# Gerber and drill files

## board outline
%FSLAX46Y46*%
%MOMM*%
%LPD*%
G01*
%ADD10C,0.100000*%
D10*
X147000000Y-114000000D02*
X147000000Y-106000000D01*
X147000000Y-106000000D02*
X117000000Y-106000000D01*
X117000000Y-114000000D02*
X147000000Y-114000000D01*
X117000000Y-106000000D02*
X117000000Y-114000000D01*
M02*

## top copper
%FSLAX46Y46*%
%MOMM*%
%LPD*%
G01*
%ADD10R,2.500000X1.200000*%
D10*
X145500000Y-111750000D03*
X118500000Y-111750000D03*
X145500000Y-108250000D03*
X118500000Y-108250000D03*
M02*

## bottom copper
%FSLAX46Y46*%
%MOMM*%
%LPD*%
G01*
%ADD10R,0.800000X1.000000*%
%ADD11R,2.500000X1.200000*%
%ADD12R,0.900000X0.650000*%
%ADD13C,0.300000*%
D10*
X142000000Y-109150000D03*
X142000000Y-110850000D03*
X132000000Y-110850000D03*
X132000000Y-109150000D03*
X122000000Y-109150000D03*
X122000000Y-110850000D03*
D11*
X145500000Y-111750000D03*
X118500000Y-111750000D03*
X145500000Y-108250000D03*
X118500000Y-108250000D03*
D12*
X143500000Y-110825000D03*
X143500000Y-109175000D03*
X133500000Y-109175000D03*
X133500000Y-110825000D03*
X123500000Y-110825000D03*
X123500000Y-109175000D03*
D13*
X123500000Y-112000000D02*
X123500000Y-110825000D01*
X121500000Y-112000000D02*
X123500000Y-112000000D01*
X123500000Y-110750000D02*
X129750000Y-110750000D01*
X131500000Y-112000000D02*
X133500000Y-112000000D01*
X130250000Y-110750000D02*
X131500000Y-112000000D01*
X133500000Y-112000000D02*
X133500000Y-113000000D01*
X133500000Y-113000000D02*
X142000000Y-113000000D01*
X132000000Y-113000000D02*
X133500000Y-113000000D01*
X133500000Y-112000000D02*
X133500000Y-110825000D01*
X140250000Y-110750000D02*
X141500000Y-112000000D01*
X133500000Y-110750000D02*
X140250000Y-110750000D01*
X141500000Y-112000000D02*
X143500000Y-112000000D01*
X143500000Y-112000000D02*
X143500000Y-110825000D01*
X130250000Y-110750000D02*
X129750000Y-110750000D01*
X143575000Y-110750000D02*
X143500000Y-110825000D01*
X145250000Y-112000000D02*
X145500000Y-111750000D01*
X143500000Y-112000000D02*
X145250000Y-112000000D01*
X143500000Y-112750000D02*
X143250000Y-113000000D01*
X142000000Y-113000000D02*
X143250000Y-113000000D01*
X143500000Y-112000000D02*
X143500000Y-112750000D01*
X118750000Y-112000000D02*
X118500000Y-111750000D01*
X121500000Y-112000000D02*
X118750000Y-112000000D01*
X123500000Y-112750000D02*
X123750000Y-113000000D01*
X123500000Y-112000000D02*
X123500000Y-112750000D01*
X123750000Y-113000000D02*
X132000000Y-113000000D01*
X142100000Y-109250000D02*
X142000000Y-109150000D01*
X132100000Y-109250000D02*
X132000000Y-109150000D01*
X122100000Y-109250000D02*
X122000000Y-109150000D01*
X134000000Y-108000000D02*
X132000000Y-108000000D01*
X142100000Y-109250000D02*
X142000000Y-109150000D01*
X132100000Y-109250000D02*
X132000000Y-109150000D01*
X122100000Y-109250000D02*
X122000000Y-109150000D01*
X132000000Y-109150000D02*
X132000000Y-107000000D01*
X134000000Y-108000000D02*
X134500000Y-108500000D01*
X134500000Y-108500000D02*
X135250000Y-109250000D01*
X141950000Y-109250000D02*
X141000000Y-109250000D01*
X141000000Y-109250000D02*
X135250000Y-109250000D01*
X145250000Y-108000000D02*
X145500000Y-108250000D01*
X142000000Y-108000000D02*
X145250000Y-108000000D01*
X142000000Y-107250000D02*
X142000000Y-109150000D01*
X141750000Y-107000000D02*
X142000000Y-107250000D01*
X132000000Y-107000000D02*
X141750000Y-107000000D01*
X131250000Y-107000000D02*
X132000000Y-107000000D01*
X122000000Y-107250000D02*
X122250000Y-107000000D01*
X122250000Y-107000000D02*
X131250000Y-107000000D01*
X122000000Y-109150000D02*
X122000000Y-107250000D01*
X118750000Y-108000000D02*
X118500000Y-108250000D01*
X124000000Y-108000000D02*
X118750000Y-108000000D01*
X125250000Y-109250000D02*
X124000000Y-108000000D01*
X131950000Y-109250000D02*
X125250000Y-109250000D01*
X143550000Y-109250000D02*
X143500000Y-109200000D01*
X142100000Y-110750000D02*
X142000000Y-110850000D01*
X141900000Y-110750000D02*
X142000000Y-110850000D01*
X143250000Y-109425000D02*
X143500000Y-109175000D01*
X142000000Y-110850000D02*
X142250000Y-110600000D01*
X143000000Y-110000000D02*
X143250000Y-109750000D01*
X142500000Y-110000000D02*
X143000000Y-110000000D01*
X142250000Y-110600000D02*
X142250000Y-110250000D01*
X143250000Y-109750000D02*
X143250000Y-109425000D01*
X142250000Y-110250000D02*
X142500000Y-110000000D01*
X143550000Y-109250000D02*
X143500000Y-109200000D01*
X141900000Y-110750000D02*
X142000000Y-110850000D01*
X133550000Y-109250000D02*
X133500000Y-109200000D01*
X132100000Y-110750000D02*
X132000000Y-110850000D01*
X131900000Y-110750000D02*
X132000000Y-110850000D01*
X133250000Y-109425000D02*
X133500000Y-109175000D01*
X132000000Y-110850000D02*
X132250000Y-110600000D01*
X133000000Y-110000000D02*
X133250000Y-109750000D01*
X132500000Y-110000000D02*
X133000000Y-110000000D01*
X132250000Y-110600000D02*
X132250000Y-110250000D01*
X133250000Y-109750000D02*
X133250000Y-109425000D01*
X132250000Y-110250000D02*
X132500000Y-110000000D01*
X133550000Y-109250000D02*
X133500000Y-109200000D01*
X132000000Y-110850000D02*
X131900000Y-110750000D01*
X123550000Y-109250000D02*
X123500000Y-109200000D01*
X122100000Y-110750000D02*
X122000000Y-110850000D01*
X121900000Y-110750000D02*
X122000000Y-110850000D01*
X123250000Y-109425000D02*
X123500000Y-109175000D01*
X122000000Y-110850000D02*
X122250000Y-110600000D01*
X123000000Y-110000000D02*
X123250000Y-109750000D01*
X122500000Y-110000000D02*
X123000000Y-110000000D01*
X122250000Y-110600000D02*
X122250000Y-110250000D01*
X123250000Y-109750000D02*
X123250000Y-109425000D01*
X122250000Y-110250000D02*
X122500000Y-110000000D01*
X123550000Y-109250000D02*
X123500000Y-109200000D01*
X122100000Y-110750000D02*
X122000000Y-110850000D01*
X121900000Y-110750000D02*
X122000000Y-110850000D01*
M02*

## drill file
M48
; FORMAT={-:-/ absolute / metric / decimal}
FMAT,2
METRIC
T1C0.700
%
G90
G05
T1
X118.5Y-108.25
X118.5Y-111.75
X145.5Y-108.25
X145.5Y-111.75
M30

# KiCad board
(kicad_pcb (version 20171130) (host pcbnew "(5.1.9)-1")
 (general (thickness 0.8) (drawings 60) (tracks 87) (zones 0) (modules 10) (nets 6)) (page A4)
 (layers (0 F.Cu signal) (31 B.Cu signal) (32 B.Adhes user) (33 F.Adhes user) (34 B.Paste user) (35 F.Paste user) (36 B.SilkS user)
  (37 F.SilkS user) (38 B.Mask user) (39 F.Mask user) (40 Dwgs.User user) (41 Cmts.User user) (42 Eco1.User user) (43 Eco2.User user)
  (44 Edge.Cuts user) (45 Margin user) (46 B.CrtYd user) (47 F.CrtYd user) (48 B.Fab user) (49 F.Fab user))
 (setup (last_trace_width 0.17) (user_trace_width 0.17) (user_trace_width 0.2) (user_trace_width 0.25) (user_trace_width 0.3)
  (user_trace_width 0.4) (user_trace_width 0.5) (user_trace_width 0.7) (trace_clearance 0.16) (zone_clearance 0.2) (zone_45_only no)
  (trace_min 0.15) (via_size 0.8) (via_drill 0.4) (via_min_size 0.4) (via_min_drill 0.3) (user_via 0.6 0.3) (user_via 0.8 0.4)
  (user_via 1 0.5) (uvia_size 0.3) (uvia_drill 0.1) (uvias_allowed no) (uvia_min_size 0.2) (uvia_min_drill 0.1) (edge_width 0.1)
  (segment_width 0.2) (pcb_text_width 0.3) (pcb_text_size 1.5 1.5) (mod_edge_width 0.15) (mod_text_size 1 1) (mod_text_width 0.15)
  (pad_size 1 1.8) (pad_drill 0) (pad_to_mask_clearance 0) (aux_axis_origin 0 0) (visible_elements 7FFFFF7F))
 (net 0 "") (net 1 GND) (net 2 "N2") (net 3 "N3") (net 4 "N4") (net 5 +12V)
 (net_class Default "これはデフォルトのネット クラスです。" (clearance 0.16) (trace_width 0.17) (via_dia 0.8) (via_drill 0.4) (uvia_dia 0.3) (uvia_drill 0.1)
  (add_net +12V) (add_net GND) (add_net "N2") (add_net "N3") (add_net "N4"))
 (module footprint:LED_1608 (layer B.Cu) (at 142 110 270)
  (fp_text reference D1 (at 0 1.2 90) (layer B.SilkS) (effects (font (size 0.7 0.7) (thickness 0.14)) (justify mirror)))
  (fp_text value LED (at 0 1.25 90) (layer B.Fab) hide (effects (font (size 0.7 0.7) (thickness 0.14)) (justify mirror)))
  (pad 1 smd rect (at -0.85 0 270) (size 1 0.8) (layers B.Cu B.Paste B.Mask) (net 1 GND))
  (pad 2 smd rect (at 0.85 0 270) (size 1 0.8) (layers B.Cu B.Paste B.Mask) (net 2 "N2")))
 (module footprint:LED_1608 (layer B.Cu) (at 132 110 270)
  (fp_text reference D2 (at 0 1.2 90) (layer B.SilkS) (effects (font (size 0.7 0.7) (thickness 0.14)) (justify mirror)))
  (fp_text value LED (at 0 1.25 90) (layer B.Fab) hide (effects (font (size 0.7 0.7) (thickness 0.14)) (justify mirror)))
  (pad 2 smd rect (at 0.85 0 270) (size 1 0.8) (layers B.Cu B.Paste B.Mask) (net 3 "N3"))
  (pad 1 smd rect (at -0.85 0 270) (size 1 0.8) (layers B.Cu B.Paste B.Mask) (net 1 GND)))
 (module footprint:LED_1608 (layer B.Cu) (at 122 110 270)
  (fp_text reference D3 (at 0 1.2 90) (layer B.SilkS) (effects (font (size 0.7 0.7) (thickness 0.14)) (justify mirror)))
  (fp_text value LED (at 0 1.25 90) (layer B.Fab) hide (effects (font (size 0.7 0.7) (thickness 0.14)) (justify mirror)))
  (pad 1 smd rect (at -0.85 0 270) (size 1 0.8) (layers B.Cu B.Paste B.Mask) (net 1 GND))
  (pad 2 smd rect (at 0.85 0 270) (size 1 0.8) (layers B.Cu B.Paste B.Mask) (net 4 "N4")))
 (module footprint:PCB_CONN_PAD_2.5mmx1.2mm (layer F.Cu) (at 145.5 111.75)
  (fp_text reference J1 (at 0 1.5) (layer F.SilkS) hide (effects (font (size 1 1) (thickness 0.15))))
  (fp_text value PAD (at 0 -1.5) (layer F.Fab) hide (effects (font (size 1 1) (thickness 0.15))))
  (pad 1 thru_hole rect (at 0 0) (size 2.5 1.2) (drill 0.7) (layers *.Cu *.Mask) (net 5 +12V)))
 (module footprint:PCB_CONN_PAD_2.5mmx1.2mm (layer F.Cu) (at 118.5 111.75)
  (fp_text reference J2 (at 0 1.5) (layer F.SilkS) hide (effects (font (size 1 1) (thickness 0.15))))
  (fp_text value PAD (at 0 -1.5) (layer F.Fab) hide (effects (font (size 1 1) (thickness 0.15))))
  (pad 1 thru_hole rect (at 0 0) (size 2.5 1.2) (drill 0.7) (layers *.Cu *.Mask) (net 5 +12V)))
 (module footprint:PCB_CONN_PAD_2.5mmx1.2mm (layer F.Cu) (at 145.5 108.25)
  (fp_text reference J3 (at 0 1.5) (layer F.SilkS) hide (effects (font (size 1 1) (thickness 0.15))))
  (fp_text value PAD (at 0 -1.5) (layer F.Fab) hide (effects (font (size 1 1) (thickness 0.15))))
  (pad 1 thru_hole rect (at 0 0) (size 2.5 1.2) (drill 0.7) (layers *.Cu *.Mask) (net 1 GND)))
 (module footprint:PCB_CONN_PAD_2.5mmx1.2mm (layer F.Cu) (at 118.5 108.25)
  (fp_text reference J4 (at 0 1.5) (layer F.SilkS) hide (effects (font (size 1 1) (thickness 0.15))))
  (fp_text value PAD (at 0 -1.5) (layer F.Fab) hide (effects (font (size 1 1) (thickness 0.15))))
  (pad 1 thru_hole rect (at 0 0) (size 2.5 1.2) (drill 0.7) (layers *.Cu *.Mask) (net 1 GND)))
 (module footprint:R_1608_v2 (layer B.Cu) (at 143.5 110 90)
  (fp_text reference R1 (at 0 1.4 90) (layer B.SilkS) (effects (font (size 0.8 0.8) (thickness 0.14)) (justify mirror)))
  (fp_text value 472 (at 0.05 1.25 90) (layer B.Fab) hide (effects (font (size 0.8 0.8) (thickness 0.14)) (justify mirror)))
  (pad 1 smd rect (at -0.825 0 90) (size 0.65 0.9) (layers B.Cu B.Paste B.Mask) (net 5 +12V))
  (pad 2 smd rect (at 0.825 0 90) (size 0.65 0.9) (layers B.Cu B.Paste B.Mask) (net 2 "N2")))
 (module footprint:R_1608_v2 (layer B.Cu) (at 133.5 110 90)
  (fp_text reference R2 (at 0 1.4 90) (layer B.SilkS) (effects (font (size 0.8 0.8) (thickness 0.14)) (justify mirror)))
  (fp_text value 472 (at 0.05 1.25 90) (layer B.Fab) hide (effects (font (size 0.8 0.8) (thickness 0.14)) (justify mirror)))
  (pad 2 smd rect (at 0.825 0 90) (size 0.65 0.9) (layers B.Cu B.Paste B.Mask) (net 3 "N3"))
  (pad 1 smd rect (at -0.825 0 90) (size 0.65 0.9) (layers B.Cu B.Paste B.Mask) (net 5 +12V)))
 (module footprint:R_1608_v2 (layer B.Cu) (at 123.5 110 90)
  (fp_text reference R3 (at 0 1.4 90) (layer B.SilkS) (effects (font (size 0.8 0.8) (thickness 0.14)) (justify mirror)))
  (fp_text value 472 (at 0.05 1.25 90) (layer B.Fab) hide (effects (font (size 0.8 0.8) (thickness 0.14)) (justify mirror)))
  (pad 1 smd rect (at -0.825 0 90) (size 0.65 0.9) (layers B.Cu B.Paste B.Mask) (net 5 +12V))
  (pad 2 smd rect (at 0.825 0 90) (size 0.65 0.9) (layers B.Cu B.Paste B.Mask) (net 4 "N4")))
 (gr_line (start 147 114) (end 147 106) (layer Edge.Cuts) (width 0.1))
 (gr_line (start 147 106) (end 117 106) (layer Edge.Cuts) (width 0.1))
 (gr_line (start 117 114) (end 147 114) (layer Edge.Cuts) (width 0.1))
 (gr_line (start 117 106) (end 117 114) (layer Edge.Cuts) (width 0.1))
 (segment (start 123.5 112) (end 123.5 110.825) (width 0.3) (layer B.Cu) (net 5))
 (segment (start 121.5 112) (end 123.5 112) (width 0.3) (layer B.Cu) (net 5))
 (segment (start 123.5 110.75) (end 129.75 110.75) (width 0.3) (layer B.Cu) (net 5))
 (segment (start 131.5 112) (end 133.5 112) (width 0.3) (layer B.Cu) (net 5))
 (segment (start 130.25 110.75) (end 131.5 112) (width 0.3) (layer B.Cu) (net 5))
 (segment (start 133.5 112) (end 133.5 113) (width 0.3) (layer B.Cu) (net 5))
 (segment (start 133.5 113) (end 142 113) (width 0.3) (layer B.Cu) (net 5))
 (segment (start 132 113) (end 133.5 113) (width 0.3) (layer B.Cu) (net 5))
 (segment (start 133.5 112) (end 133.5 110.825) (width 0.3) (layer B.Cu) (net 5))
 (segment (start 140.25 110.75) (end 141.5 112) (width 0.3) (layer B.Cu) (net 5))
 (segment (start 133.5 110.75) (end 140.25 110.75) (width 0.3) (layer B.Cu) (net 5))
 (segment (start 141.5 112) (end 143.5 112) (width 0.3) (layer B.Cu) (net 5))
 (segment (start 143.5 112) (end 143.5 110.825) (width 0.3) (layer B.Cu) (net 5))
 (segment (start 130.25 110.75) (end 129.75 110.75) (width 0.3) (layer B.Cu) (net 5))
 (segment (start 143.575 110.75) (end 143.5 110.825) (width 0.3) (layer B.Cu) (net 5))
 (segment (start 145.25 112) (end 145.5 111.75) (width 0.3) (layer B.Cu) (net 5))
 (segment (start 143.5 112) (end 145.25 112) (width 0.3) (layer B.Cu) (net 5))
 (segment (start 143.5 112.75) (end 143.25 113) (width 0.3) (layer B.Cu) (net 5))
 (segment (start 142 113) (end 143.25 113) (width 0.3) (layer B.Cu) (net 5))
 (segment (start 143.5 112) (end 143.5 112.75) (width 0.3) (layer B.Cu) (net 5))
 (segment (start 118.75 112) (end 118.5 111.75) (width 0.3) (layer B.Cu) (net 5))
 (segment (start 121.5 112) (end 118.75 112) (width 0.3) (layer B.Cu) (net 5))
 (segment (start 123.5 112.75) (end 123.75 113) (width 0.3) (layer B.Cu) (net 5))
 (segment (start 123.5 112) (end 123.5 112.75) (width 0.3) (layer B.Cu) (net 5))
 (segment (start 123.75 113) (end 132 113) (width 0.3) (layer B.Cu) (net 5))
 (segment (start 142.1 109.25) (end 142 109.15) (width 0.3) (layer B.Cu) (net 1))
 (segment (start 132.1 109.25) (end 132 109.15) (width 0.3) (layer B.Cu) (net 1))
 (segment (start 122.1 109.25) (end 122 109.15) (width 0.3) (layer B.Cu) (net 1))
 (segment (start 134 108) (end 132 108) (width 0.3) (layer B.Cu) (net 1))
 (segment (start 142.1 109.25) (end 142 109.15) (width 0.3) (layer B.Cu) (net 1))
 (segment (start 132.1 109.25) (end 132 109.15) (width 0.3) (layer B.Cu) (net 1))
 (segment (start 122.1 109.25) (end 122 109.15) (width 0.3) (layer B.Cu) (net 1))
 (segment (start 132 109.15) (end 132 107) (width 0.3) (layer B.Cu) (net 1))
 (segment (start 134 108) (end 134.5 108.5) (width 0.3) (layer B.Cu) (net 1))
 (segment (start 134.5 108.5) (end 135.25 109.25) (width 0.3) (layer B.Cu) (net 1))
 (segment (start 141.95 109.25) (end 141 109.25) (width 0.3) (layer B.Cu) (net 1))
 (segment (start 141 109.25) (end 135.25 109.25) (width 0.3) (layer B.Cu) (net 1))
 (segment (start 145.25 108) (end 145.5 108.25) (width 0.3) (layer B.Cu) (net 1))
 (segment (start 142 108) (end 145.25 108) (width 0.3) (layer B.Cu) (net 1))
 (segment (start 142 107.25) (end 142 109.15) (width 0.3) (layer B.Cu) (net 1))
 (segment (start 141.75 107) (end 142 107.25) (width 0.3) (layer B.Cu) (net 1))
 (segment (start 132 107) (end 141.75 107) (width 0.3) (layer B.Cu) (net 1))
 (segment (start 131.25 107) (end 132 107) (width 0.3) (layer B.Cu) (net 1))
 (segment (start 122 107.25) (end 122.25 107) (width 0.3) (layer B.Cu) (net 1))
 (segment (start 122.25 107) (end 131.25 107) (width 0.3) (layer B.Cu) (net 1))
 (segment (start 122 109.15) (end 122 107.25) (width 0.3) (layer B.Cu) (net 1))
 (segment (start 118.75 108) (end 118.5 108.25) (width 0.3) (layer B.Cu) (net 1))
 (segment (start 124 108) (end 118.75 108) (width 0.3) (layer B.Cu) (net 1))
 (segment (start 125.25 109.25) (end 124 108) (width 0.3) (layer B.Cu) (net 1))
 (segment (start 131.95 109.25) (end 125.25 109.25) (width 0.3) (layer B.Cu) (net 1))
 (segment (start 143.55 109.25) (end 143.5 109.2) (width 0.3) (layer B.Cu) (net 2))
 (segment (start 142.1 110.75) (end 142 110.85) (width 0.3) (layer B.Cu) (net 2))
 (segment (start 141.9 110.75) (end 142 110.85) (width 0.3) (layer B.Cu) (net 2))
 (segment (start 143.25 109.425) (end 143.5 109.175) (width 0.3) (layer B.Cu) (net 2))
 (segment (start 142 110.85) (end 142.25 110.6) (width 0.3) (layer B.Cu) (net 2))
 (segment (start 143 110) (end 143.25 109.75) (width 0.3) (layer B.Cu) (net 2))
 (segment (start 142.5 110) (end 143 110) (width 0.3) (layer B.Cu) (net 2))
 (segment (start 142.25 110.6) (end 142.25 110.25) (width 0.3) (layer B.Cu) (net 2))
 (segment (start 143.25 109.75) (end 143.25 109.425) (width 0.3) (layer B.Cu) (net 2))
 (segment (start 142.25 110.25) (end 142.5 110) (width 0.3) (layer B.Cu) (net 2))
 (segment (start 143.55 109.25) (end 143.5 109.2) (width 0.3) (layer B.Cu) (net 2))
 (segment (start 141.9 110.75) (end 142 110.85) (width 0.3) (layer B.Cu) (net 2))
 (segment (start 133.55 109.25) (end 133.5 109.2) (width 0.3) (layer B.Cu) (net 3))
 (segment (start 132.1 110.75) (end 132 110.85) (width 0.3) (layer B.Cu) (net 3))
 (segment (start 131.9 110.75) (end 132 110.85) (width 0.3) (layer B.Cu) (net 3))
 (segment (start 133.25 109.425) (end 133.5 109.175) (width 0.3) (layer B.Cu) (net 3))
 (segment (start 132 110.85) (end 132.25 110.6) (width 0.3) (layer B.Cu) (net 3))
 (segment (start 133 110) (end 133.25 109.75) (width 0.3) (layer B.Cu) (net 3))
 (segment (start 132.5 110) (end 133 110) (width 0.3) (layer B.Cu) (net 3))
 (segment (start 132.25 110.6) (end 132.25 110.25) (width 0.3) (layer B.Cu) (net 3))
 (segment (start 133.25 109.75) (end 133.25 109.425) (width 0.3) (layer B.Cu) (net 3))
 (segment (start 132.25 110.25) (end 132.5 110) (width 0.3) (layer B.Cu) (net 3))
 (segment (start 133.55 109.25) (end 133.5 109.2) (width 0.3) (layer B.Cu) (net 3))
 (segment (start 132 110.85) (end 131.9 110.75) (width 0.3) (layer B.Cu) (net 3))
 (segment (start 123.55 109.25) (end 123.5 109.2) (width 0.3) (layer B.Cu) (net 4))
 (segment (start 122.1 110.75) (end 122 110.85) (width 0.3) (layer B.Cu) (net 4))
 (segment (start 121.9 110.75) (end 122 110.85) (width 0.3) (layer B.Cu) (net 4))
 (segment (start 123.25 109.425) (end 123.5 109.175) (width 0.3) (layer B.Cu) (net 4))
 (segment (start 122 110.85) (end 122.25 110.6) (width 0.3) (layer B.Cu) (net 4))
 (segment (start 123 110) (end 123.25 109.75) (width 0.3) (layer B.Cu) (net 4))
 (segment (start 122.5 110) (end 123 110) (width 0.3) (layer B.Cu) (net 4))
 (segment (start 122.25 110.6) (end 122.25 110.25) (width 0.3) (layer B.Cu) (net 4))
 (segment (start 123.25 109.75) (end 123.25 109.425) (width 0.3) (layer B.Cu) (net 4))
 (segment (start 122.25 110.25) (end 122.5 110) (width 0.3) (layer B.Cu) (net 4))
 (segment (start 123.55 109.25) (end 123.5 109.2) (width 0.3) (layer B.Cu) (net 4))
 (segment (start 122.1 110.75) (end 122 110.85) (width 0.3) (layer B.Cu) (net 4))
 (segment (start 121.9 110.75) (end 122 110.85) (width 0.3) (layer B.Cu) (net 4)))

